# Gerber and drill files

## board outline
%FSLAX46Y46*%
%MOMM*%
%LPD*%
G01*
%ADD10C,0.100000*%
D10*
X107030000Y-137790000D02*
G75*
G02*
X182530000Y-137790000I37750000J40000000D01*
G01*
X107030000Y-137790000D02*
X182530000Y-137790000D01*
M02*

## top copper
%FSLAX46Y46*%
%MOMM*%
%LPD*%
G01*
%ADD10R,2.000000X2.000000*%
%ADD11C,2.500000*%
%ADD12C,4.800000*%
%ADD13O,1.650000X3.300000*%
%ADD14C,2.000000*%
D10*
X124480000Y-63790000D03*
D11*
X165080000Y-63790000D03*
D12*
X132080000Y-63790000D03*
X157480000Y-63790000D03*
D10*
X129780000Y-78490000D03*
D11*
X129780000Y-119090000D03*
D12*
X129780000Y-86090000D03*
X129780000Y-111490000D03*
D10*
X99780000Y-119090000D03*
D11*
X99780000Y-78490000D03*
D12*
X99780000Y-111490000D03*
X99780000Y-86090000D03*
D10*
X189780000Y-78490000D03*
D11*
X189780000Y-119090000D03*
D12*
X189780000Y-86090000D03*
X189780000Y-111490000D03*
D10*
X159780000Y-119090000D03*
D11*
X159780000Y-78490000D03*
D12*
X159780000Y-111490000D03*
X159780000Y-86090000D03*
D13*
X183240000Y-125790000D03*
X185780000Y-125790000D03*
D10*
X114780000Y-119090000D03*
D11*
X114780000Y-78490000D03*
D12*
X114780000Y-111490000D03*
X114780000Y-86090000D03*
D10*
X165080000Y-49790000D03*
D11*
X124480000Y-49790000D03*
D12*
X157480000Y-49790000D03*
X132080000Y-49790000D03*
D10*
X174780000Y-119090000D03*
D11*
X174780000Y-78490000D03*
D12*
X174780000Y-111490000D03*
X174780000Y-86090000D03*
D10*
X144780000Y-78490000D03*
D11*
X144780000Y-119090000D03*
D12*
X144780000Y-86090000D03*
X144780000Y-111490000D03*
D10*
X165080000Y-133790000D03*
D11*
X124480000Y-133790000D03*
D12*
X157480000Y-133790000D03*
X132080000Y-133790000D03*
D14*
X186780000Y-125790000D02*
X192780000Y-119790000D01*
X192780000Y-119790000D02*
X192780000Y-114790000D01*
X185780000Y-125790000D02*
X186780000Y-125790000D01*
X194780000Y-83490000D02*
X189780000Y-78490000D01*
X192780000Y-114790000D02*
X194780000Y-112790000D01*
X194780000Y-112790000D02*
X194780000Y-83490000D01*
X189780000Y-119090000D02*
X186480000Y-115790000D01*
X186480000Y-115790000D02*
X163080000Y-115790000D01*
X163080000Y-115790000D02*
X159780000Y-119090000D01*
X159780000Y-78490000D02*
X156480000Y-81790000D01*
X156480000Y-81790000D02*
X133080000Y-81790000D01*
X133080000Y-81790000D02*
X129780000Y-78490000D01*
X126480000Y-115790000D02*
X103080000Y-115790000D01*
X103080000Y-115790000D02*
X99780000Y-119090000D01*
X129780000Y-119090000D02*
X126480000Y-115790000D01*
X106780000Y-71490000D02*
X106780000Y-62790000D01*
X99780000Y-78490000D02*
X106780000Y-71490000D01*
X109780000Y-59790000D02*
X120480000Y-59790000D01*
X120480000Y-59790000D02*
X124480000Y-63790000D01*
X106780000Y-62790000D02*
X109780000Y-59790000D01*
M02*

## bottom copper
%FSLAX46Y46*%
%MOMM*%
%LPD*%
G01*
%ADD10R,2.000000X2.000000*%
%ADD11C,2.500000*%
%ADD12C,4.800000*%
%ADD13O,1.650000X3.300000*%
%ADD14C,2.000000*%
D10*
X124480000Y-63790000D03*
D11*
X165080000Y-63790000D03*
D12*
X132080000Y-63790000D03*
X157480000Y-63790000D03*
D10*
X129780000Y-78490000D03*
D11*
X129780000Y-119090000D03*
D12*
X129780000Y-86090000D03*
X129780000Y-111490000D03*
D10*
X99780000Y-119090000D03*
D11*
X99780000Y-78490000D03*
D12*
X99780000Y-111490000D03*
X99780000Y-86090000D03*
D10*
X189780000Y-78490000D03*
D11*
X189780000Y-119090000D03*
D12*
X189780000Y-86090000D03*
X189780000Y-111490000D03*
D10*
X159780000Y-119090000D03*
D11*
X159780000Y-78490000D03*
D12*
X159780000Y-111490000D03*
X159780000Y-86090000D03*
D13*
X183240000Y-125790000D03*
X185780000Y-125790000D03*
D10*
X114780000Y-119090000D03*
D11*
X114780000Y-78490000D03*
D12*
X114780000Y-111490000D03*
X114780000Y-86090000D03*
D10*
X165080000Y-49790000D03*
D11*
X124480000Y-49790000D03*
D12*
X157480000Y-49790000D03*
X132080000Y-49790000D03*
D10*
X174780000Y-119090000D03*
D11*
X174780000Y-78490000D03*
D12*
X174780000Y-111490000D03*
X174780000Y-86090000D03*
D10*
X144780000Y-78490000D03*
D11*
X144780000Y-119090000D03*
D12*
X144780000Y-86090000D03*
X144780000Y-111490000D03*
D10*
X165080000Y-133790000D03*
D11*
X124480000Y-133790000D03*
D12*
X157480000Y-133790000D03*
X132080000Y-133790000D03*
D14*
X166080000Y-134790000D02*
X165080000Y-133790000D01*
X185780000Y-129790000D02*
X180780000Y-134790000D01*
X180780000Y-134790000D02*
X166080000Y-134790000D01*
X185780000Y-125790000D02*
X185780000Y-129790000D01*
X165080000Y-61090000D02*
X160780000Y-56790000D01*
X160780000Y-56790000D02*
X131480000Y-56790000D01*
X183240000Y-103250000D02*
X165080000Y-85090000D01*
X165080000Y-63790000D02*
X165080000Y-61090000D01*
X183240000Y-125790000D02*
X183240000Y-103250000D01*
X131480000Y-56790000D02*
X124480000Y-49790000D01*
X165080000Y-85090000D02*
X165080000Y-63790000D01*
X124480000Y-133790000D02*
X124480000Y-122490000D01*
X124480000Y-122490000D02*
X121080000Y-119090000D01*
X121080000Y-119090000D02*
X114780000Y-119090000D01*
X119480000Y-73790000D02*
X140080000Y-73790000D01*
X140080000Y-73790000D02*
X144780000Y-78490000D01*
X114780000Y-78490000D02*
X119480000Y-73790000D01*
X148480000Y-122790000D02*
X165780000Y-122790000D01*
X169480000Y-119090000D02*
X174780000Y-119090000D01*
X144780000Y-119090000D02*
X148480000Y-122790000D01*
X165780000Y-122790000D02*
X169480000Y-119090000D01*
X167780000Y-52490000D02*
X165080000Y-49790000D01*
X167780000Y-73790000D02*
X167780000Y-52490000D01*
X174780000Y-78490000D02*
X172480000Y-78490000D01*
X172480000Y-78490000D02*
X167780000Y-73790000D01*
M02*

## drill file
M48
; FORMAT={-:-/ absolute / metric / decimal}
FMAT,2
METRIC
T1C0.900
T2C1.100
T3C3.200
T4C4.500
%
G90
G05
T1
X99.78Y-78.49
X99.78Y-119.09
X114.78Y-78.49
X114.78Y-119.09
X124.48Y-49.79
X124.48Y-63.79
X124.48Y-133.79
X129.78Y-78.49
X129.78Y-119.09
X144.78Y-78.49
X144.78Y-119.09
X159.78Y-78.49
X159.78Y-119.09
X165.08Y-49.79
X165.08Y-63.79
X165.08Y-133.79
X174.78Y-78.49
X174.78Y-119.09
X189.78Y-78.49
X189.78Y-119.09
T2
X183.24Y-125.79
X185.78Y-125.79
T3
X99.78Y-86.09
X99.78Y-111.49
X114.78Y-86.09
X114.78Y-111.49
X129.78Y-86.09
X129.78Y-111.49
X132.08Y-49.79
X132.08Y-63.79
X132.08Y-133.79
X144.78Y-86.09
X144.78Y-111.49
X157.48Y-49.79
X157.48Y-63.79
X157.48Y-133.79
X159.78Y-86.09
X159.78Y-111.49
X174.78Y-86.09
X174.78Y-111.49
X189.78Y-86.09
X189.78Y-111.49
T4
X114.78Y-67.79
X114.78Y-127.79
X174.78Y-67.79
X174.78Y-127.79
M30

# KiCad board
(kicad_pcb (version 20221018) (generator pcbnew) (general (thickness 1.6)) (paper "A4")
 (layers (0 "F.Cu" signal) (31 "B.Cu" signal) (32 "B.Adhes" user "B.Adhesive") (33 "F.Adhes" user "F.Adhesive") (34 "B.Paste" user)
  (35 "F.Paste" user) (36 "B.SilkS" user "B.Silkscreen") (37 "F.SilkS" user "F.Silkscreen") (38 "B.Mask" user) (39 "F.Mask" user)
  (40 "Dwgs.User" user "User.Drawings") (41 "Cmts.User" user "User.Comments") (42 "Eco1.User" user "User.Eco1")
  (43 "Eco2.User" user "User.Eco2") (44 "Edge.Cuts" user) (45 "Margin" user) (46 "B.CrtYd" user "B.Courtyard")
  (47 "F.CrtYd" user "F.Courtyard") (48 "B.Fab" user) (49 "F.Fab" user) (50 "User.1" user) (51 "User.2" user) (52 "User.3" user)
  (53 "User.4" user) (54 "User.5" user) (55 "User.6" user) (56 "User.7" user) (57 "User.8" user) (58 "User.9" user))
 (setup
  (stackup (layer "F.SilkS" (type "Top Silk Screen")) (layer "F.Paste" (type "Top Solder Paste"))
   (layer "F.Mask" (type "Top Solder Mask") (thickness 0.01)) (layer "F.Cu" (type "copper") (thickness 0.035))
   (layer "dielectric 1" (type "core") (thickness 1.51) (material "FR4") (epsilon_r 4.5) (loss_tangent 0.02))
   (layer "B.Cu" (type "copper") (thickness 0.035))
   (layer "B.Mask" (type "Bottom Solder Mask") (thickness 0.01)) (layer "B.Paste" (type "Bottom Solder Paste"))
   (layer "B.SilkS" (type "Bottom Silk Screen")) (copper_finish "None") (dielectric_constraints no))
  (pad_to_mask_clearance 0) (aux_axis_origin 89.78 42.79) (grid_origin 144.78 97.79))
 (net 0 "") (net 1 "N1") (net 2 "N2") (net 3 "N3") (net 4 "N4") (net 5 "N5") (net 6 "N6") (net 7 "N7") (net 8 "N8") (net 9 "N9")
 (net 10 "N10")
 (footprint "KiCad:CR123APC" (layer "F.Cu") (at 124.48 63.79)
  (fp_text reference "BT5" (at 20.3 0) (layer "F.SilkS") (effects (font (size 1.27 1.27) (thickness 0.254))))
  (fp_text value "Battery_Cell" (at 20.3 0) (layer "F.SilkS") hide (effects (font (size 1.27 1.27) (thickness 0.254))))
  (pad "1" thru_hole rect (at 0 0) (size 2 2) (drill 0.9) (layers "*.Cu" "*.Mask") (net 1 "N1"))
  (pad "2" thru_hole circle (at 40.6 0) (size 2.5 2.5) (drill 0.9) (layers "*.Cu" "*.Mask") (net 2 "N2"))
  (pad "MH1" thru_hole circle (at 7.6 0) (size 4.8 4.8) (drill 3.2) (layers "*.Cu" "*.Mask"))
  (pad "MH2" thru_hole circle (at 33 0) (size 4.8 4.8) (drill 3.2) (layers "*.Cu" "*.Mask")))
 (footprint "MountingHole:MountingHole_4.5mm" (layer "F.Cu") (at 174.78 127.79)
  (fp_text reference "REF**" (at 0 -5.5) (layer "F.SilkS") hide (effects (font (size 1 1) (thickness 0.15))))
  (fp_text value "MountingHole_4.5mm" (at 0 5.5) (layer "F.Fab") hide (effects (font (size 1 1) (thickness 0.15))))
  (pad "" np_thru_hole circle (at 0 0) (size 4.5 4.5) (drill 4.5) (layers "*.Cu" "*.Mask")))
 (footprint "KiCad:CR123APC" (layer "F.Cu") (at 129.78 78.49 -90)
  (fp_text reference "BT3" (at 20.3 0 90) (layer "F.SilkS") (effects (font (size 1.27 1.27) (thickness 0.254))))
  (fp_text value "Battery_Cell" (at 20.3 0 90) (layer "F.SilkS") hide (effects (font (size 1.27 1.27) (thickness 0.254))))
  (pad "1" thru_hole rect (at 0 0 270) (size 2 2) (drill 0.9) (layers "*.Cu" "*.Mask") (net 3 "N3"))
  (pad "2" thru_hole circle (at 40.6 0 270) (size 2.5 2.5) (drill 0.9) (layers "*.Cu" "*.Mask") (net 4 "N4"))
  (pad "MH1" thru_hole circle (at 7.6 0 270) (size 4.8 4.8) (drill 3.2) (layers "*.Cu" "*.Mask"))
  (pad "MH2" thru_hole circle (at 33 0 270) (size 4.8 4.8) (drill 3.2) (layers "*.Cu" "*.Mask")))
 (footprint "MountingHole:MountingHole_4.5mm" (layer "F.Cu") (at 174.78 67.79)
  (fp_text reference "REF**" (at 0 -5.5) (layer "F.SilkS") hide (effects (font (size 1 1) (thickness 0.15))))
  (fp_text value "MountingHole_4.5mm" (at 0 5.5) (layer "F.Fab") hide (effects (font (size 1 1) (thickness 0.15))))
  (pad "" np_thru_hole circle (at 0 0) (size 4.5 4.5) (drill 4.5) (layers "*.Cu" "*.Mask")))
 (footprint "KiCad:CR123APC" (layer "F.Cu") (at 99.78 119.09 90)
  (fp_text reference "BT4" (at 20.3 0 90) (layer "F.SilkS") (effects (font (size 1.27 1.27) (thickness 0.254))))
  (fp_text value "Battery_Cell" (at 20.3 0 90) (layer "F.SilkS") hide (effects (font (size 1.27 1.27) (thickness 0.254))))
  (pad "1" thru_hole rect (at 0 0 90) (size 2 2) (drill 0.9) (layers "*.Cu" "*.Mask") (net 4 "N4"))
  (pad "2" thru_hole circle (at 40.6 0 90) (size 2.5 2.5) (drill 0.9) (layers "*.Cu" "*.Mask") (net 1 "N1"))
  (pad "MH1" thru_hole circle (at 7.6 0 90) (size 4.8 4.8) (drill 3.2) (layers "*.Cu" "*.Mask"))
  (pad "MH2" thru_hole circle (at 33 0 90) (size 4.8 4.8) (drill 3.2) (layers "*.Cu" "*.Mask")))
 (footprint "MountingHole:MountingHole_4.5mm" (layer "F.Cu") (at 114.78 67.79)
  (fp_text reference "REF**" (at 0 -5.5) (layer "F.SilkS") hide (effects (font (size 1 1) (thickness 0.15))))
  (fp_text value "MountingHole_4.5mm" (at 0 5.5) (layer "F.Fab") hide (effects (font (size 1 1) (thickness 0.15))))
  (pad "" np_thru_hole circle (at 0 0) (size 4.5 4.5) (drill 4.5) (layers "*.Cu" "*.Mask")))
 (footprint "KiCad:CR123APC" (layer "F.Cu") (at 189.78 78.49 -90)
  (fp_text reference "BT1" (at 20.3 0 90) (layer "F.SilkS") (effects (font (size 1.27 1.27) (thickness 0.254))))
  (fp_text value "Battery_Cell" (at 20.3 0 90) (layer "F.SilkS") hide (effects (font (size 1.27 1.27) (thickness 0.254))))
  (pad "1" thru_hole rect (at 0 0 270) (size 2 2) (drill 0.9) (layers "*.Cu" "*.Mask") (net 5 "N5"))
  (pad "2" thru_hole circle (at 40.6 0 270) (size 2.5 2.5) (drill 0.9) (layers "*.Cu" "*.Mask") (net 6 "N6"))
  (pad "MH1" thru_hole circle (at 7.6 0 270) (size 4.8 4.8) (drill 3.2) (layers "*.Cu" "*.Mask"))
  (pad "MH2" thru_hole circle (at 33 0 270) (size 4.8 4.8) (drill 3.2) (layers "*.Cu" "*.Mask")))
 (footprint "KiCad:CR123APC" (layer "F.Cu") (at 159.78 119.09 90)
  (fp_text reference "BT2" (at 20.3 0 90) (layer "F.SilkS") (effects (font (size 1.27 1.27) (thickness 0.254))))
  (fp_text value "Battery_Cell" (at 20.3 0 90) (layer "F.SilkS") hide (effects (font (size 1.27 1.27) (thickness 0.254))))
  (pad "1" thru_hole rect (at 0 0 90) (size 2 2) (drill 0.9) (layers "*.Cu" "*.Mask") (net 6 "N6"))
  (pad "2" thru_hole circle (at 40.6 0 90) (size 2.5 2.5) (drill 0.9) (layers "*.Cu" "*.Mask") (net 3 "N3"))
  (pad "MH1" thru_hole circle (at 7.6 0 90) (size 4.8 4.8) (drill 3.2) (layers "*.Cu" "*.Mask"))
  (pad "MH2" thru_hole circle (at 33 0 90) (size 4.8 4.8) (drill 3.2) (layers "*.Cu" "*.Mask")))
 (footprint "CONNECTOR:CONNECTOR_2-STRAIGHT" (layer "F.Cu") (at 184.51 125.79)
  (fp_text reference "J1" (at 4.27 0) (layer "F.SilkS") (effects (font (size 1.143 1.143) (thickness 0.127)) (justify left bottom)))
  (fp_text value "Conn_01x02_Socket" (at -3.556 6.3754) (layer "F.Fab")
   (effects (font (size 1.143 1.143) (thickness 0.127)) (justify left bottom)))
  (pad "1" thru_hole oval (at -1.27 0 90) (size 3.3 1.65) (drill 1.1) (layers "*.Cu" "*.Mask") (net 2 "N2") (solder_mask_margin 0.1016)
   (thermal_bridge_angle 45))
  (pad "2" thru_hole oval (at 1.27 0 90) (size 3.3 1.65) (drill 1.1) (layers "*.Cu" "*.Mask") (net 5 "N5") (solder_mask_margin 0.1016)
   (thermal_bridge_angle 45)))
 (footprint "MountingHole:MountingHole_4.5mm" (layer "F.Cu") (at 114.78 127.79)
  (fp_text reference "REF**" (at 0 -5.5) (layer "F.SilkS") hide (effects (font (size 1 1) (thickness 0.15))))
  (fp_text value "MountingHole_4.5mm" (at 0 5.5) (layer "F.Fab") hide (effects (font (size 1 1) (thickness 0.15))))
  (pad "" np_thru_hole circle (at 0 0) (size 4.5 4.5) (drill 4.5) (layers "*.Cu" "*.Mask")))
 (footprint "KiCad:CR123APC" (layer "B.Cu") (at 114.78 119.09 90)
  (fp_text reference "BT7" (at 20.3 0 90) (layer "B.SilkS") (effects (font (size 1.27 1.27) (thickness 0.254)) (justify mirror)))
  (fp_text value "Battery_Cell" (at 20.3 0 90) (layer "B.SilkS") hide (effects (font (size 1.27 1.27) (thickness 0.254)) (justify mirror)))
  (pad "1" thru_hole rect (at 0 0 90) (size 2 2) (drill 0.9) (layers "*.Cu" "*.Mask") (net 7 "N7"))
  (pad "2" thru_hole circle (at 40.6 0 90) (size 2.5 2.5) (drill 0.9) (layers "*.Cu" "*.Mask") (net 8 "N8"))
  (pad "MH1" thru_hole circle (at 7.6 0 90) (size 4.8 4.8) (drill 3.2) (layers "*.Cu" "*.Mask"))
  (pad "MH2" thru_hole circle (at 33 0 90) (size 4.8 4.8) (drill 3.2) (layers "*.Cu" "*.Mask")))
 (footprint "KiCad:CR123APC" (layer "B.Cu") (at 165.08 49.79 180)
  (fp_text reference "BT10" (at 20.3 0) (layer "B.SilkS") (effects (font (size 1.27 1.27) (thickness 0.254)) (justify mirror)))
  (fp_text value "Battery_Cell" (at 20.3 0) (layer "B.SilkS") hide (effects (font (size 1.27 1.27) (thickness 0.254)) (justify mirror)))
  (pad "1" thru_hole rect (at 0 0 180) (size 2 2) (drill 0.9) (layers "*.Cu" "*.Mask") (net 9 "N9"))
  (pad "2" thru_hole circle (at 40.6 0 180) (size 2.5 2.5) (drill 0.9) (layers "*.Cu" "*.Mask") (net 2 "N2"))
  (pad "MH1" thru_hole circle (at 7.6 0 180) (size 4.8 4.8) (drill 3.2) (layers "*.Cu" "*.Mask"))
  (pad "MH2" thru_hole circle (at 33 0 180) (size 4.8 4.8) (drill 3.2) (layers "*.Cu" "*.Mask")))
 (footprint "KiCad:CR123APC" (layer "B.Cu") (at 174.78 119.09 90)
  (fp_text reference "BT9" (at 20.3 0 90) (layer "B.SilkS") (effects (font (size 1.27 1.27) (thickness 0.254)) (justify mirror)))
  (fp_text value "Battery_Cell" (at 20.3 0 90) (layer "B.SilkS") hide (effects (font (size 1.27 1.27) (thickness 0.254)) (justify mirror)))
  (pad "1" thru_hole rect (at 0 0 90) (size 2 2) (drill 0.9) (layers "*.Cu" "*.Mask") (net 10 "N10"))
  (pad "2" thru_hole circle (at 40.6 0 90) (size 2.5 2.5) (drill 0.9) (layers "*.Cu" "*.Mask") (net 9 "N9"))
  (pad "MH1" thru_hole circle (at 7.6 0 90) (size 4.8 4.8) (drill 3.2) (layers "*.Cu" "*.Mask"))
  (pad "MH2" thru_hole circle (at 33 0 90) (size 4.8 4.8) (drill 3.2) (layers "*.Cu" "*.Mask")))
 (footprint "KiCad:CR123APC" (layer "B.Cu") (at 144.78 78.49 -90)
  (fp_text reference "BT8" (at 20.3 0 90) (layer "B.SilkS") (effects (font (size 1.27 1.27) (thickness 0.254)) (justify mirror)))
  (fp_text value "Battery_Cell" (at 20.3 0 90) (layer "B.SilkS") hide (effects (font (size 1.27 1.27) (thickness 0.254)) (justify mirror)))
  (pad "1" thru_hole rect (at 0 0 270) (size 2 2) (drill 0.9) (layers "*.Cu" "*.Mask") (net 8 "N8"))
  (pad "2" thru_hole circle (at 40.6 0 270) (size 2.5 2.5) (drill 0.9) (layers "*.Cu" "*.Mask") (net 10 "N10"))
  (pad "MH1" thru_hole circle (at 7.6 0 270) (size 4.8 4.8) (drill 3.2) (layers "*.Cu" "*.Mask"))
  (pad "MH2" thru_hole circle (at 33 0 270) (size 4.8 4.8) (drill 3.2) (layers "*.Cu" "*.Mask")))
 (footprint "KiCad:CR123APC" (layer "B.Cu") (at 165.08 133.79 180)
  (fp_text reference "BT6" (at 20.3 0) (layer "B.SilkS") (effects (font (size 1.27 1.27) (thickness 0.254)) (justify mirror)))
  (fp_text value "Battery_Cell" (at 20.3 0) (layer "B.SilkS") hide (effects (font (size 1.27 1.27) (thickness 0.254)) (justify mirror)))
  (pad "1" thru_hole rect (at 0 0 180) (size 2 2) (drill 0.9) (layers "*.Cu" "*.Mask") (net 5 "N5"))
  (pad "2" thru_hole circle (at 40.6 0 180) (size 2.5 2.5) (drill 0.9) (layers "*.Cu" "*.Mask") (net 7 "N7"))
  (pad "MH1" thru_hole circle (at 7.6 0 180) (size 4.8 4.8) (drill 3.2) (layers "*.Cu" "*.Mask"))
  (pad "MH2" thru_hole circle (at 33 0 180) (size 4.8 4.8) (drill 3.2) (layers "*.Cu" "*.Mask")))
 (gr_arc (start 107.03 137.79) (mid 144.78 42.789432) (end 182.53 137.79) (stroke (width 0.1) (type default)) (layer "Edge.Cuts"))
 (gr_line (start 107.03 137.79) (end 182.53 137.79) (stroke (width 0.1) (type default)) (layer "Edge.Cuts"))
 (segment (start 186.78 125.79) (end 192.78 119.79) (width 2) (layer "F.Cu") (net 5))
 (segment (start 192.78 119.79) (end 192.78 114.79) (width 2) (layer "F.Cu") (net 5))
 (segment (start 185.78 125.79) (end 186.78 125.79) (width 2) (layer "F.Cu") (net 5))
 (segment (start 194.78 83.49) (end 189.78 78.49) (width 2) (layer "F.Cu") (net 5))
 (segment (start 192.78 114.79) (end 194.78 112.79) (width 2) (layer "F.Cu") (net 5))
 (segment (start 194.78 112.79) (end 194.78 83.49) (width 2) (layer "F.Cu") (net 5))
 (segment (start 166.08 134.79) (end 165.08 133.79) (width 2) (layer "B.Cu") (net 5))
 (segment (start 185.78 129.79) (end 180.78 134.79) (width 2) (layer "B.Cu") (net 5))
 (segment (start 180.78 134.79) (end 166.08 134.79) (width 2) (layer "B.Cu") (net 5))
 (segment (start 185.78 125.79) (end 185.78 129.79) (width 2) (layer "B.Cu") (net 5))
 (segment (start 189.78 119.09) (end 186.48 115.79) (width 2) (layer "F.Cu") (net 6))
 (segment (start 186.48 115.79) (end 163.08 115.79) (width 2) (layer "F.Cu") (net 6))
 (segment (start 163.08 115.79) (end 159.78 119.09) (width 2) (layer "F.Cu") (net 6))
 (segment (start 159.78 78.49) (end 156.48 81.79) (width 2) (layer "F.Cu") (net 3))
 (segment (start 156.48 81.79) (end 133.08 81.79) (width 2) (layer "F.Cu") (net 3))
 (segment (start 133.08 81.79) (end 129.78 78.49) (width 2) (layer "F.Cu") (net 3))
 (segment (start 126.48 115.79) (end 103.08 115.79) (width 2) (layer "F.Cu") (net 4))
 (segment (start 103.08 115.79) (end 99.78 119.09) (width 2) (layer "F.Cu") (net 4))
 (segment (start 129.78 119.09) (end 126.48 115.79) (width 2) (layer "F.Cu") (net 4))
 (segment (start 106.78 71.49) (end 106.78 62.79) (width 2) (layer "F.Cu") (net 1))
 (segment (start 99.78 78.49) (end 106.78 71.49) (width 2) (layer "F.Cu") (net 1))
 (segment (start 109.78 59.79) (end 120.48 59.79) (width 2) (layer "F.Cu") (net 1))
 (segment (start 120.48 59.79) (end 124.48 63.79) (width 2) (layer "F.Cu") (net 1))
 (segment (start 106.78 62.79) (end 109.78 59.79) (width 2) (layer "F.Cu") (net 1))
 (segment (start 165.08 61.09) (end 160.78 56.79) (width 2) (layer "B.Cu") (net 2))
 (segment (start 160.78 56.79) (end 131.48 56.79) (width 2) (layer "B.Cu") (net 2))
 (segment (start 183.24 103.25) (end 165.08 85.09) (width 2) (layer "B.Cu") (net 2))
 (segment (start 165.08 63.79) (end 165.08 61.09) (width 2) (layer "B.Cu") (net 2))
 (segment (start 183.24 125.79) (end 183.24 103.25) (width 2) (layer "B.Cu") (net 2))
 (segment (start 131.48 56.79) (end 124.48 49.79) (width 2) (layer "B.Cu") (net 2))
 (segment (start 165.08 85.09) (end 165.08 63.79) (width 2) (layer "B.Cu") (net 2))
 (segment (start 124.48 133.79) (end 124.48 122.49) (width 2) (layer "B.Cu") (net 7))
 (segment (start 124.48 122.49) (end 121.08 119.09) (width 2) (layer "B.Cu") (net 7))
 (segment (start 121.08 119.09) (end 114.78 119.09) (width 2) (layer "B.Cu") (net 7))
 (segment (start 119.48 73.79) (end 140.08 73.79) (width 2) (layer "B.Cu") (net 8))
 (segment (start 140.08 73.79) (end 144.78 78.49) (width 2) (layer "B.Cu") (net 8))
 (segment (start 114.78 78.49) (end 119.48 73.79) (width 2) (layer "B.Cu") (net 8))
 (segment (start 148.48 122.79) (end 165.78 122.79) (width 2) (layer "B.Cu") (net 10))
 (segment (start 169.48 119.09) (end 174.78 119.09) (width 2) (layer "B.Cu") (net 10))
 (segment (start 144.78 119.09) (end 148.48 122.79) (width 2) (layer "B.Cu") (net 10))
 (segment (start 165.78 122.79) (end 169.48 119.09) (width 2) (layer "B.Cu") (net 10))
 (segment (start 167.78 52.49) (end 165.08 49.79) (width 2) (layer "B.Cu") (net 9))
 (segment (start 167.78 73.79) (end 167.78 52.49) (width 2) (layer "B.Cu") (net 9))
 (segment (start 174.78 78.49) (end 172.48 78.49) (width 2) (layer "B.Cu") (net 9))
 (segment (start 172.48 78.49) (end 167.78 73.79) (width 2) (layer "B.Cu") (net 9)))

